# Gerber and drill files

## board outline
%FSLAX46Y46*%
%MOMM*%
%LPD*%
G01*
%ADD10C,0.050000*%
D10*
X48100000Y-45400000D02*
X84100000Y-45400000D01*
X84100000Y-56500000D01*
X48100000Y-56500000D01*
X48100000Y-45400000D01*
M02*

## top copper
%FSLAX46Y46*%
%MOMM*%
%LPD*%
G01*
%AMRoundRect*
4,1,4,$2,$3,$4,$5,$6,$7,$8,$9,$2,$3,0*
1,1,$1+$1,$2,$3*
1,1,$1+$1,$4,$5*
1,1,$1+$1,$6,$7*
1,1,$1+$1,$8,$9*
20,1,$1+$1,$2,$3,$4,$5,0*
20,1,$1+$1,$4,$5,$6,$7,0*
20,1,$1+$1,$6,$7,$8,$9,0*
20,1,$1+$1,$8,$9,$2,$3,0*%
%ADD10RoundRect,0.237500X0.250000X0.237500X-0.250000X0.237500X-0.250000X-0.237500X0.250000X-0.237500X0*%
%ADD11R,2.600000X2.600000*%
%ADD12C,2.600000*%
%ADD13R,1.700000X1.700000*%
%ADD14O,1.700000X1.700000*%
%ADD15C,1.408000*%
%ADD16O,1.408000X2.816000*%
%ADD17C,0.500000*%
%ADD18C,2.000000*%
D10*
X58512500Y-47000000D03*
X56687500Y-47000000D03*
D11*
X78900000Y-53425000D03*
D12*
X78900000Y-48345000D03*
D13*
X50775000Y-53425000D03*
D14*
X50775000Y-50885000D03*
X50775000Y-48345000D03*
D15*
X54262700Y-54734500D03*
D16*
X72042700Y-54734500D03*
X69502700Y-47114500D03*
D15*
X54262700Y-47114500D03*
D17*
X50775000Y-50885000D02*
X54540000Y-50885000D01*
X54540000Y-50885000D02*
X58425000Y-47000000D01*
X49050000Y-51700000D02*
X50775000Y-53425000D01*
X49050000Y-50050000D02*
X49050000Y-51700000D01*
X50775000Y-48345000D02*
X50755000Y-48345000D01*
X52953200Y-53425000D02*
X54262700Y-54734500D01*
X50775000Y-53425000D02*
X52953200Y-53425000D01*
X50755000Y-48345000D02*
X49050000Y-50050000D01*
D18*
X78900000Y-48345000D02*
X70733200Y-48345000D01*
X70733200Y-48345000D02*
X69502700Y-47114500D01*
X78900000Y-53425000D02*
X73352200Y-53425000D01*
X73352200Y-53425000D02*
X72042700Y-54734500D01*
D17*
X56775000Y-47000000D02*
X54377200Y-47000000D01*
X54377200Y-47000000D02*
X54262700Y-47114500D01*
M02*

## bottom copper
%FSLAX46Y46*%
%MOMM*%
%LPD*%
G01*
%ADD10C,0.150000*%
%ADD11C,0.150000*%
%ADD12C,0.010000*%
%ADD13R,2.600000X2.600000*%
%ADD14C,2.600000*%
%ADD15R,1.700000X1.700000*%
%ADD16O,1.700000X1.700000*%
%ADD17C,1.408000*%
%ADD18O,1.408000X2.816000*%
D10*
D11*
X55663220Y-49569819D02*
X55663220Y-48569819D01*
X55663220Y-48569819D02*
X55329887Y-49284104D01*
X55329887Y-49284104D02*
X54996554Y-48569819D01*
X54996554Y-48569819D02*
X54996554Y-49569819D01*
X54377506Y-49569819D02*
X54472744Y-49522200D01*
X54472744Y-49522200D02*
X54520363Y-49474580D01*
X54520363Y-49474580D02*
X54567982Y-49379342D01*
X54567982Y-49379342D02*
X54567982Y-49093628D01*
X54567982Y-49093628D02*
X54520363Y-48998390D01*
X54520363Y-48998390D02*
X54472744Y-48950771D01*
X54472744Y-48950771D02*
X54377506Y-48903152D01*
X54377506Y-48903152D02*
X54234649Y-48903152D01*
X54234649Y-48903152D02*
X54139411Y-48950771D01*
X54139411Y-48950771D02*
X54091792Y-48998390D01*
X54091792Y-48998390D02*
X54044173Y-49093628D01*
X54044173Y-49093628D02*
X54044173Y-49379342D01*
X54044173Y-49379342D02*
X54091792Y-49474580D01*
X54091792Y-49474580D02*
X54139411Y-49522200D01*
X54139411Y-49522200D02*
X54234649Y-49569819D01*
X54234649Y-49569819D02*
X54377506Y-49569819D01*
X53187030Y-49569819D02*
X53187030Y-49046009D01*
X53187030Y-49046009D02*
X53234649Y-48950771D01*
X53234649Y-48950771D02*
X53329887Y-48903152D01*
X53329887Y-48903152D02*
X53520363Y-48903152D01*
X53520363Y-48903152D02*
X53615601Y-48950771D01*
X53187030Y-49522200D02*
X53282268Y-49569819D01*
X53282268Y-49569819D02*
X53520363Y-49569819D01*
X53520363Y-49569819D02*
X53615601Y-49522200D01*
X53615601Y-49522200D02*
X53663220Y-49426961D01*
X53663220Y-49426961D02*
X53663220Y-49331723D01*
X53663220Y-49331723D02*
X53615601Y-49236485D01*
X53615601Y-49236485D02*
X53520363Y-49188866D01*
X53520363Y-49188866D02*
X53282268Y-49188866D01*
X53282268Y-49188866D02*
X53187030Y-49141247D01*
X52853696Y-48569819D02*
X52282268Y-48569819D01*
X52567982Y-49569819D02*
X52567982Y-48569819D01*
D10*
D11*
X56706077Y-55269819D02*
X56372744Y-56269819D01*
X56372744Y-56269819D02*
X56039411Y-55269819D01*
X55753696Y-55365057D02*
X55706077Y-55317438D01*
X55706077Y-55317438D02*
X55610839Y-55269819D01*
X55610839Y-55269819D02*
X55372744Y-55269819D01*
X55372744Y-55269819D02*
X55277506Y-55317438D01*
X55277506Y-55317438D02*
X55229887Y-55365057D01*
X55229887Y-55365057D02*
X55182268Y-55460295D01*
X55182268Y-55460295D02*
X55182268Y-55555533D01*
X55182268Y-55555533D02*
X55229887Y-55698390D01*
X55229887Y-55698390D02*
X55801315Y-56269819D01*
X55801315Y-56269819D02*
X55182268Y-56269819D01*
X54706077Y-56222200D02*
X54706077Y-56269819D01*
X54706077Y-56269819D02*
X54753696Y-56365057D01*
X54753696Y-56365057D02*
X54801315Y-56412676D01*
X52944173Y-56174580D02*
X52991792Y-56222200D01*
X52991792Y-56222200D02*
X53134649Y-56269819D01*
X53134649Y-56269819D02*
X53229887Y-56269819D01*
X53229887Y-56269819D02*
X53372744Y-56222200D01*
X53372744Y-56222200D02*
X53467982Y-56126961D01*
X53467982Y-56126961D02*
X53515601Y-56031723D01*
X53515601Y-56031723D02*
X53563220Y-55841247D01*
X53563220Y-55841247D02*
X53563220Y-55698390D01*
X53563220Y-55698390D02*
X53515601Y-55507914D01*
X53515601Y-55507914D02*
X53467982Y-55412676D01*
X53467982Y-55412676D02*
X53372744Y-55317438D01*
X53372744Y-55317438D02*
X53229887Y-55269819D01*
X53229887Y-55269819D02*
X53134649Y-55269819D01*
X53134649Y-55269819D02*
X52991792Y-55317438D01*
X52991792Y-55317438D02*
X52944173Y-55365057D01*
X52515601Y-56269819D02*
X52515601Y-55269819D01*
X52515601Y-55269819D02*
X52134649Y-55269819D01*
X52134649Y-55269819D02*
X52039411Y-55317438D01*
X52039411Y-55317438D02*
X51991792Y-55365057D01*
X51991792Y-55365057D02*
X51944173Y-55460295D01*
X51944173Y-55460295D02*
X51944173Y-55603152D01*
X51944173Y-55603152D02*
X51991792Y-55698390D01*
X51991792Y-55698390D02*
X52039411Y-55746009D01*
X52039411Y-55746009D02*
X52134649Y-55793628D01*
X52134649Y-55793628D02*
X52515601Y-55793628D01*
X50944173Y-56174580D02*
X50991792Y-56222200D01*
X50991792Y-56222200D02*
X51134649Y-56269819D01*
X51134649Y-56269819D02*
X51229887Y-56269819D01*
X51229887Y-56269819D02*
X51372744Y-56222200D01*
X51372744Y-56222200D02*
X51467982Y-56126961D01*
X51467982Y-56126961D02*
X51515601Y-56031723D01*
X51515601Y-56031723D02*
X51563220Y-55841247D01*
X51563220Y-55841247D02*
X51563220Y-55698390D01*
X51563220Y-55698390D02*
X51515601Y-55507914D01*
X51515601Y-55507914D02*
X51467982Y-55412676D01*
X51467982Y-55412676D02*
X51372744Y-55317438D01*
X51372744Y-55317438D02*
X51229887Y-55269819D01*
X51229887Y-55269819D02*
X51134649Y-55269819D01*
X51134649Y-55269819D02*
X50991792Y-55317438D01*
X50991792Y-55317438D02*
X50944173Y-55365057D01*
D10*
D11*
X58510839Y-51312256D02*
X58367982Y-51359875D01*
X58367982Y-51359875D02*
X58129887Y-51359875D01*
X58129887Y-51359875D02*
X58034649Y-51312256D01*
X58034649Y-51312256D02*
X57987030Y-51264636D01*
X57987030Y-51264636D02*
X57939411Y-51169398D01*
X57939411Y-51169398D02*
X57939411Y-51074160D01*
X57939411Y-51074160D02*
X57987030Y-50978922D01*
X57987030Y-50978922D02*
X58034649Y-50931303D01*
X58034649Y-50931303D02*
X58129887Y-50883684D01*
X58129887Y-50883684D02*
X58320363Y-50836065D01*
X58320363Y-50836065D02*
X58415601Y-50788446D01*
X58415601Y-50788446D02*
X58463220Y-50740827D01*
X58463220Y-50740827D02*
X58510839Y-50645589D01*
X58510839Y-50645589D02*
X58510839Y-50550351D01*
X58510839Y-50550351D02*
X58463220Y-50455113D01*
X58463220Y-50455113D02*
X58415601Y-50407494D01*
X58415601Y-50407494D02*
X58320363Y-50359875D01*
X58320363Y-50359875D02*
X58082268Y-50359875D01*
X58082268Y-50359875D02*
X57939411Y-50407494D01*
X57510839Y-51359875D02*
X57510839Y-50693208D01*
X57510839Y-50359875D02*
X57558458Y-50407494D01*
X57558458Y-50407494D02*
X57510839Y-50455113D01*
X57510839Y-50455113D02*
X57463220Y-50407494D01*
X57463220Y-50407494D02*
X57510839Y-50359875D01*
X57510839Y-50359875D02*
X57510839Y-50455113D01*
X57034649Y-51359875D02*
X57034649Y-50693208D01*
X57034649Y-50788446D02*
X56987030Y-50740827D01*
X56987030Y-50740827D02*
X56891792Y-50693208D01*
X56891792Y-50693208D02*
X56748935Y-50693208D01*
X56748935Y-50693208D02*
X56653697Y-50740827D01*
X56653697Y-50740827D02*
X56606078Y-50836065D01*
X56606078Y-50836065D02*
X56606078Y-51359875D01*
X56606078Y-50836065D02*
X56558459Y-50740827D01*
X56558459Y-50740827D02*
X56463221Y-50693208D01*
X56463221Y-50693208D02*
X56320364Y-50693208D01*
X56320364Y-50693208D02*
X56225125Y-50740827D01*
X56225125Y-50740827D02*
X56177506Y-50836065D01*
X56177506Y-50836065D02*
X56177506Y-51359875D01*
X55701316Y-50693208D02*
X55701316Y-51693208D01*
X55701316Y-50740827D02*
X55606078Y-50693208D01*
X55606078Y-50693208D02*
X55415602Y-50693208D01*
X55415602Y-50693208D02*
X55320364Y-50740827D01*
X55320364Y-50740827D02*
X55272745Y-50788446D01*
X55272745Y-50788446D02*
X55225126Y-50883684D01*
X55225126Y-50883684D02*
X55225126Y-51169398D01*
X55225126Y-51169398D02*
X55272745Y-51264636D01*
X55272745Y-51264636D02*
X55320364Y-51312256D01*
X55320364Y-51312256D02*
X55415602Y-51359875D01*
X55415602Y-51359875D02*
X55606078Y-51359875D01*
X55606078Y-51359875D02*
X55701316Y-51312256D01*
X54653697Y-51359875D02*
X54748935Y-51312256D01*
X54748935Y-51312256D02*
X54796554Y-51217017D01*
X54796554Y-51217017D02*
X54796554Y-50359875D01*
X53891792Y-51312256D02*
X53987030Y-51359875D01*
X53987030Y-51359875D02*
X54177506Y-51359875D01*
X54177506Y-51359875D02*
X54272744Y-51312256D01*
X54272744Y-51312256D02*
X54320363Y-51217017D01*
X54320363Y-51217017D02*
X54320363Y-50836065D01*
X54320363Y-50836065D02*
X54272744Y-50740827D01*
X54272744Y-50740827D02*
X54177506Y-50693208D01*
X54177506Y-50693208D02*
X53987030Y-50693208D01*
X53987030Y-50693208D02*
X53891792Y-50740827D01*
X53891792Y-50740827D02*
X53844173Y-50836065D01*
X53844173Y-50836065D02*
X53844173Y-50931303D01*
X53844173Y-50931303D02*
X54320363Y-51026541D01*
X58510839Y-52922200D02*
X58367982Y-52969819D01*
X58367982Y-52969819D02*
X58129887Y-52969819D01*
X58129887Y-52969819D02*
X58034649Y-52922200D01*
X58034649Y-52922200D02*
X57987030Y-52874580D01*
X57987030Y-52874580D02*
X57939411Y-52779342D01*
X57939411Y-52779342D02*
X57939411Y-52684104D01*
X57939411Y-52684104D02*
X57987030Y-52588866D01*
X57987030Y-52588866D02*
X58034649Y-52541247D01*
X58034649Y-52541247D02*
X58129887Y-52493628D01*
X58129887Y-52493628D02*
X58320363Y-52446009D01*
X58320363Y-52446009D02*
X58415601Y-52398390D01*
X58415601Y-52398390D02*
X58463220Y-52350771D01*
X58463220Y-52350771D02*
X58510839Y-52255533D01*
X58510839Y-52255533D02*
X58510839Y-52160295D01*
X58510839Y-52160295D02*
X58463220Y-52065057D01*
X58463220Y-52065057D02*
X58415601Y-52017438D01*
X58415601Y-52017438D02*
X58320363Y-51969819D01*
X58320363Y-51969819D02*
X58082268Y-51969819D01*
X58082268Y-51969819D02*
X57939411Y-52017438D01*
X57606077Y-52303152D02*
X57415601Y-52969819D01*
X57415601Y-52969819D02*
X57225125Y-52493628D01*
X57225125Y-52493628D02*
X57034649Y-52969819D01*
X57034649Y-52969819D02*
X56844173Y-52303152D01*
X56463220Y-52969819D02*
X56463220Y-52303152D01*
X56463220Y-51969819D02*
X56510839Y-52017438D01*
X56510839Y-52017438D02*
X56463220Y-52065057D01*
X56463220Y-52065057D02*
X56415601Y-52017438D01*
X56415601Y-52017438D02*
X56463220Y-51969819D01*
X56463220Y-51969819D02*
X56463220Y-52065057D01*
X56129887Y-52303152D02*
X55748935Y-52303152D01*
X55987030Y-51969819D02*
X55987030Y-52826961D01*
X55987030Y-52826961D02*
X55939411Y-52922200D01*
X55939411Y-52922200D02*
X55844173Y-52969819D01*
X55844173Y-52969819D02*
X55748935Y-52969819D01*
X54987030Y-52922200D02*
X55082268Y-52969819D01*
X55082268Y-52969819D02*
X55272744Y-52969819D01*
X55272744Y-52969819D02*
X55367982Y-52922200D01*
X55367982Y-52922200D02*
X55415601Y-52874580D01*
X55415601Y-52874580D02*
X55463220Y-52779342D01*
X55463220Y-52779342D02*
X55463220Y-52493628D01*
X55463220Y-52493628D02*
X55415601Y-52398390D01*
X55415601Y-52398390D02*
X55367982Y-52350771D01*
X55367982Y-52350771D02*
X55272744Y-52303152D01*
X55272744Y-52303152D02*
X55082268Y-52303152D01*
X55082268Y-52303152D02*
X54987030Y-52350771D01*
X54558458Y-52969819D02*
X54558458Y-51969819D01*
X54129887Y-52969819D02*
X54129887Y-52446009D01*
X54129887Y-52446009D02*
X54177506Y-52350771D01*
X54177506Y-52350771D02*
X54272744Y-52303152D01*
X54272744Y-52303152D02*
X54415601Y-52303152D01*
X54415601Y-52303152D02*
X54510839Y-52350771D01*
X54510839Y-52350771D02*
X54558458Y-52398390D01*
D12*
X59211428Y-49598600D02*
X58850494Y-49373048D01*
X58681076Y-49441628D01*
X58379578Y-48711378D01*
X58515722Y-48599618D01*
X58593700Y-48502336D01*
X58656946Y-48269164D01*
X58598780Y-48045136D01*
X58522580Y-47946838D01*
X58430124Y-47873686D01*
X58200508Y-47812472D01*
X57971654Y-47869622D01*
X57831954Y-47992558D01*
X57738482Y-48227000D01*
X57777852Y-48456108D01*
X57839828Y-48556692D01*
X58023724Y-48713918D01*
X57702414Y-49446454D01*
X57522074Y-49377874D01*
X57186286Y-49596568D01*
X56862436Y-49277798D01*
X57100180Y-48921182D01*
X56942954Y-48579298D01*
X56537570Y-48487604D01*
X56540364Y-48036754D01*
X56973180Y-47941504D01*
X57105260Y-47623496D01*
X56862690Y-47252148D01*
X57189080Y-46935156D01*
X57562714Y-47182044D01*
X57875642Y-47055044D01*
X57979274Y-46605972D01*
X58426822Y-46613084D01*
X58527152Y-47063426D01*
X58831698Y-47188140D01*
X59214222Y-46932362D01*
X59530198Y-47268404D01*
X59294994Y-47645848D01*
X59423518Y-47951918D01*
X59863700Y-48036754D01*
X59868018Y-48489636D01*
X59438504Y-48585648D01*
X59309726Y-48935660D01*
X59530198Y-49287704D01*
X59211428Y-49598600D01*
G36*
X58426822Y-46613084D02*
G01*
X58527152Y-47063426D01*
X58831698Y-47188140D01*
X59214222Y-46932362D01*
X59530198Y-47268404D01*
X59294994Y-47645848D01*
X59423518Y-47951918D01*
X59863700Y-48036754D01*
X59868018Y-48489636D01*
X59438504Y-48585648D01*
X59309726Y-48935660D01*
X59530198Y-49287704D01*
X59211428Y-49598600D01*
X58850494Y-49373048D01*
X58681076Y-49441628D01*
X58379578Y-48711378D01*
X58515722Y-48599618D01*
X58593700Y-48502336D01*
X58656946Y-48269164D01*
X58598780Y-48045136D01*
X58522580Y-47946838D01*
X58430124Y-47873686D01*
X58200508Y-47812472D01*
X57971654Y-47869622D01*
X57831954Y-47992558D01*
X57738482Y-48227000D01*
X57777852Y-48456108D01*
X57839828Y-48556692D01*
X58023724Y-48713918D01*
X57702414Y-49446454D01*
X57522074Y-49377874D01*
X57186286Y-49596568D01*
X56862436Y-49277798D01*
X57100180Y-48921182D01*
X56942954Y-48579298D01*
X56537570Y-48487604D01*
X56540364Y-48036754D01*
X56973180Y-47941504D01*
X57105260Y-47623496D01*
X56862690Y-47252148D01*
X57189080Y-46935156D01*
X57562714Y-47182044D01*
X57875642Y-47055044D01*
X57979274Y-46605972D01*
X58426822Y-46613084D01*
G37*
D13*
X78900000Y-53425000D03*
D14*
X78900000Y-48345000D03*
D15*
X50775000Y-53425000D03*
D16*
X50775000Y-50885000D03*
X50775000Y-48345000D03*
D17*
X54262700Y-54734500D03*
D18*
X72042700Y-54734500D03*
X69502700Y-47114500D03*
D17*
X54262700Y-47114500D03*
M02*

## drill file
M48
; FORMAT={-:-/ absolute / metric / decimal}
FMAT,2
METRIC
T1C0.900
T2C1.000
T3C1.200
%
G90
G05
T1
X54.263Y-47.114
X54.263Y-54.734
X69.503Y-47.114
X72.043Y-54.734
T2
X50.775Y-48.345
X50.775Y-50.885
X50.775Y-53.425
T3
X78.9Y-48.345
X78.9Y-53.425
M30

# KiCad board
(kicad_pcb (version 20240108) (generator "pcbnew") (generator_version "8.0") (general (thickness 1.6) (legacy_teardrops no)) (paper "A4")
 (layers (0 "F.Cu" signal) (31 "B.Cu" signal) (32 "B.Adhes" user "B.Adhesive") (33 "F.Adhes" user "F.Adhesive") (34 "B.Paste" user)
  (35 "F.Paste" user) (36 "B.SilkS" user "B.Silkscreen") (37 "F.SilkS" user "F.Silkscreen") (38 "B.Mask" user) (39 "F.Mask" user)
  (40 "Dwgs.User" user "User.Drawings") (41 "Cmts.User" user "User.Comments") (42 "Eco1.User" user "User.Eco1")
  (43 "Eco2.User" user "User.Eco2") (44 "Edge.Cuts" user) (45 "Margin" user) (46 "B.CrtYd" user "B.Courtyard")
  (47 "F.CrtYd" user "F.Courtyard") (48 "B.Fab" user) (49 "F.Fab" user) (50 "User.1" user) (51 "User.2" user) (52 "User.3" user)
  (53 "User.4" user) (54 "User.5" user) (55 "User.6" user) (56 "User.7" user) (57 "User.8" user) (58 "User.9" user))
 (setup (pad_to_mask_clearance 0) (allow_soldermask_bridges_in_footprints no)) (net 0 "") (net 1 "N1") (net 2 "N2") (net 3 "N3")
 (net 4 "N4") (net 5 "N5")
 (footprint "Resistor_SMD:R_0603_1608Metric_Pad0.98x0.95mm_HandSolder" (layer "F.Cu") (at 57.6 47 180)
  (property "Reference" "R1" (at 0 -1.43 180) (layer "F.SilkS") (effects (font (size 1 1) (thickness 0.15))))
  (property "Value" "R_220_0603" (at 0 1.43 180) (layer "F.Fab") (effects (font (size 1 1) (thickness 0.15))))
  (pad "1" smd roundrect (at -0.9125 0 180) (size 0.975 0.95) (layers "F.Cu" "F.Paste" "F.Mask") (roundrect_rratio 0.25) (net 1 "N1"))
  (pad "2" smd roundrect (at 0.9125 0 180) (size 0.975 0.95) (layers "F.Cu" "F.Paste" "F.Mask") (roundrect_rratio 0.25) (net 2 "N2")))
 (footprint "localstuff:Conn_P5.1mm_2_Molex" (layer "F.Cu") (at 78.9 53.425 90)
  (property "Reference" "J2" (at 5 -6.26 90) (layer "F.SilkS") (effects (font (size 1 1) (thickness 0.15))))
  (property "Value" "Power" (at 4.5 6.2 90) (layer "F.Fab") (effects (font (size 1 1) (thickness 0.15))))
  (pad "1" thru_hole rect (at 0 0 90) (size 2.6 2.6) (drill 1.2) (layers "*.Cu" "*.Mask") (remove_unused_layers no) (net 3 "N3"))
  (pad "2" thru_hole circle (at 5.08 0 90) (size 2.6 2.6) (drill 1.2) (layers "*.Cu" "*.Mask") (remove_unused_layers no) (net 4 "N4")))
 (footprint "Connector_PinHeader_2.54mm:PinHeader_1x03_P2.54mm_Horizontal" (layer "F.Cu") (at 50.775 53.425 180)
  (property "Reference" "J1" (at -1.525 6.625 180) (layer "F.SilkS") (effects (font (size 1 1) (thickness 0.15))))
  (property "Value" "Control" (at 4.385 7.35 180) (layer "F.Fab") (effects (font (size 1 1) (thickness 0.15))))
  (pad "1" thru_hole rect (at 0 0 180) (size 1.7 1.7) (drill 1) (layers "*.Cu" "*.Mask") (remove_unused_layers no) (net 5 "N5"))
  (pad "2" thru_hole oval (at 0 2.54 180) (size 1.7 1.7) (drill 1) (layers "*.Cu" "*.Mask") (remove_unused_layers no) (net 1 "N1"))
  (pad "3" thru_hole oval (at 0 5.08 180) (size 1.7 1.7) (drill 1) (layers "*.Cu" "*.Mask") (remove_unused_layers no) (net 5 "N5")))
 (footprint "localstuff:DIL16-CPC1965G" (layer "F.Cu") (at 63.1527 50.9245)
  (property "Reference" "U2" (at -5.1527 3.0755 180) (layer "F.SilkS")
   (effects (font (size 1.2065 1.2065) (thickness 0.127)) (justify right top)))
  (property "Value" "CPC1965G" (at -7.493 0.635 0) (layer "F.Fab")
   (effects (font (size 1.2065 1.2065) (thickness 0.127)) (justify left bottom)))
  (pad "1" thru_hole circle (at -8.89 3.81 90) (size 1.408 1.408) (drill 0.9) (layers "*.Cu" "*.Mask") (remove_unused_layers no)
   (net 5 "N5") (solder_mask_margin 0.1016))
  (pad "8" thru_hole oval (at 8.89 3.81 90) (size 2.816 1.408) (drill 0.9) (layers "*.Cu" "*.Mask") (remove_unused_layers no) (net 3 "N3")
   (solder_mask_margin 0.1016))
  (pad "10" thru_hole oval (at 6.35 -3.81 90) (size 2.816 1.408) (drill 0.9) (layers "*.Cu" "*.Mask") (remove_unused_layers no) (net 4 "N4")
   (solder_mask_margin 0.1016))
  (pad "16" thru_hole circle (at -8.89 -3.81 90) (size 1.408 1.408) (drill 0.9) (layers "*.Cu" "*.Mask") (remove_unused_layers no)
   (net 2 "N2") (solder_mask_margin 0.1016)))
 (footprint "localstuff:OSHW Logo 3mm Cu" (layer "B.Cu") (at 58.2 48.1 180)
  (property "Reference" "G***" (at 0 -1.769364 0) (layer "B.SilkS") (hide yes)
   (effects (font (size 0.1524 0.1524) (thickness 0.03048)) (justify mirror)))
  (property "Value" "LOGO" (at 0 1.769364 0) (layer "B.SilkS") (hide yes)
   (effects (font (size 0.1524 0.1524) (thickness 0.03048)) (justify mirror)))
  (fp_poly
   (pts (xy -1.011428 -1.4986) (xy -0.650494 -1.273048) (xy -0.481076 -1.341628) (xy -0.179578 -0.611378) (xy -0.315722 -0.499618)
    (xy -0.3937 -0.402336) (xy -0.456946 -0.169164) (xy -0.39878 0.054864) (xy -0.32258 0.153162) (xy -0.230124 0.226314)
    (xy -0.000508 0.287528) (xy 0.228346 0.230378) (xy 0.368046 0.107442) (xy 0.461518 -0.127) (xy 0.422148 -0.356108)
    (xy 0.360172 -0.456692) (xy 0.176276 -0.613918) (xy 0.497586 -1.346454) (xy 0.677926 -1.277874) (xy 1.013714 -1.496568)
    (xy 1.337564 -1.177798) (xy 1.09982 -0.821182) (xy 1.257046 -0.479298) (xy 1.66243 -0.387604) (xy 1.659636 0.063246)
    (xy 1.22682 0.158496) (xy 1.09474 0.476504) (xy 1.33731 0.847852) (xy 1.01092 1.164844) (xy 0.637286 0.917956) (xy 0.324358 1.044956)
    (xy 0.220726 1.494028) (xy -0.226822 1.486916) (xy -0.327152 1.036574) (xy -0.631698 0.91186) (xy -1.014222 1.167638)
    (xy -1.330198 0.831596) (xy -1.094994 0.454152) (xy -1.223518 0.148082) (xy -1.6637 0.063246) (xy -1.668018 -0.389636)
    (xy -1.238504 -0.485648) (xy -1.109726 -0.83566) (xy -1.330198 -1.187704) (xy -1.011428 -1.4986))
   (stroke (width 0.01) (type solid)) (fill solid) (layer "B.Cu")))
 (gr_rect (start 48.1 45.4) (end 84.1 56.5) (stroke (width 0.05) (type default)) (fill none) (layer "Edge.Cuts"))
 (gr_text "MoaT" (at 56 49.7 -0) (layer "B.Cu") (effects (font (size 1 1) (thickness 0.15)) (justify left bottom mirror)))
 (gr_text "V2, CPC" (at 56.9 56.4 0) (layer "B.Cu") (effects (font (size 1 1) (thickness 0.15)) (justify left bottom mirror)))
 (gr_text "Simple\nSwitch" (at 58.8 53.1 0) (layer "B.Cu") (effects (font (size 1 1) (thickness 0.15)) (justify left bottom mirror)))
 (segment (start 50.775 50.885) (end 54.54 50.885) (width 0.5) (layer "F.Cu") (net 1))
 (segment (start 54.54 50.885) (end 58.425 47) (width 0.5) (layer "F.Cu") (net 1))
 (segment (start 49.05 51.7) (end 50.775 53.425) (width 0.5) (layer "F.Cu") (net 5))
 (segment (start 49.05 50.05) (end 49.05 51.7) (width 0.5) (layer "F.Cu") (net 5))
 (segment (start 50.775 48.345) (end 50.755 48.345) (width 0.5) (layer "F.Cu") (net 5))
 (segment (start 52.9532 53.425) (end 54.2627 54.7345) (width 0.5) (layer "F.Cu") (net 5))
 (segment (start 50.775 53.425) (end 52.9532 53.425) (width 0.5) (layer "F.Cu") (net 5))
 (segment (start 50.755 48.345) (end 49.05 50.05) (width 0.5) (layer "F.Cu") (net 5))
 (segment (start 78.9 48.345) (end 70.7332 48.345) (width 2) (layer "F.Cu") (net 4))
 (segment (start 70.7332 48.345) (end 69.5027 47.1145) (width 2) (layer "F.Cu") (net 4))
 (segment (start 78.9 53.425) (end 73.3522 53.425) (width 2) (layer "F.Cu") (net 3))
 (segment (start 73.3522 53.425) (end 72.0427 54.7345) (width 2) (layer "F.Cu") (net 3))
 (segment (start 56.775 47) (end 54.3772 47) (width 0.5) (layer "F.Cu") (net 2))
 (segment (start 54.3772 47) (end 54.2627 47.1145) (width 0.5) (layer "F.Cu") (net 2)))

